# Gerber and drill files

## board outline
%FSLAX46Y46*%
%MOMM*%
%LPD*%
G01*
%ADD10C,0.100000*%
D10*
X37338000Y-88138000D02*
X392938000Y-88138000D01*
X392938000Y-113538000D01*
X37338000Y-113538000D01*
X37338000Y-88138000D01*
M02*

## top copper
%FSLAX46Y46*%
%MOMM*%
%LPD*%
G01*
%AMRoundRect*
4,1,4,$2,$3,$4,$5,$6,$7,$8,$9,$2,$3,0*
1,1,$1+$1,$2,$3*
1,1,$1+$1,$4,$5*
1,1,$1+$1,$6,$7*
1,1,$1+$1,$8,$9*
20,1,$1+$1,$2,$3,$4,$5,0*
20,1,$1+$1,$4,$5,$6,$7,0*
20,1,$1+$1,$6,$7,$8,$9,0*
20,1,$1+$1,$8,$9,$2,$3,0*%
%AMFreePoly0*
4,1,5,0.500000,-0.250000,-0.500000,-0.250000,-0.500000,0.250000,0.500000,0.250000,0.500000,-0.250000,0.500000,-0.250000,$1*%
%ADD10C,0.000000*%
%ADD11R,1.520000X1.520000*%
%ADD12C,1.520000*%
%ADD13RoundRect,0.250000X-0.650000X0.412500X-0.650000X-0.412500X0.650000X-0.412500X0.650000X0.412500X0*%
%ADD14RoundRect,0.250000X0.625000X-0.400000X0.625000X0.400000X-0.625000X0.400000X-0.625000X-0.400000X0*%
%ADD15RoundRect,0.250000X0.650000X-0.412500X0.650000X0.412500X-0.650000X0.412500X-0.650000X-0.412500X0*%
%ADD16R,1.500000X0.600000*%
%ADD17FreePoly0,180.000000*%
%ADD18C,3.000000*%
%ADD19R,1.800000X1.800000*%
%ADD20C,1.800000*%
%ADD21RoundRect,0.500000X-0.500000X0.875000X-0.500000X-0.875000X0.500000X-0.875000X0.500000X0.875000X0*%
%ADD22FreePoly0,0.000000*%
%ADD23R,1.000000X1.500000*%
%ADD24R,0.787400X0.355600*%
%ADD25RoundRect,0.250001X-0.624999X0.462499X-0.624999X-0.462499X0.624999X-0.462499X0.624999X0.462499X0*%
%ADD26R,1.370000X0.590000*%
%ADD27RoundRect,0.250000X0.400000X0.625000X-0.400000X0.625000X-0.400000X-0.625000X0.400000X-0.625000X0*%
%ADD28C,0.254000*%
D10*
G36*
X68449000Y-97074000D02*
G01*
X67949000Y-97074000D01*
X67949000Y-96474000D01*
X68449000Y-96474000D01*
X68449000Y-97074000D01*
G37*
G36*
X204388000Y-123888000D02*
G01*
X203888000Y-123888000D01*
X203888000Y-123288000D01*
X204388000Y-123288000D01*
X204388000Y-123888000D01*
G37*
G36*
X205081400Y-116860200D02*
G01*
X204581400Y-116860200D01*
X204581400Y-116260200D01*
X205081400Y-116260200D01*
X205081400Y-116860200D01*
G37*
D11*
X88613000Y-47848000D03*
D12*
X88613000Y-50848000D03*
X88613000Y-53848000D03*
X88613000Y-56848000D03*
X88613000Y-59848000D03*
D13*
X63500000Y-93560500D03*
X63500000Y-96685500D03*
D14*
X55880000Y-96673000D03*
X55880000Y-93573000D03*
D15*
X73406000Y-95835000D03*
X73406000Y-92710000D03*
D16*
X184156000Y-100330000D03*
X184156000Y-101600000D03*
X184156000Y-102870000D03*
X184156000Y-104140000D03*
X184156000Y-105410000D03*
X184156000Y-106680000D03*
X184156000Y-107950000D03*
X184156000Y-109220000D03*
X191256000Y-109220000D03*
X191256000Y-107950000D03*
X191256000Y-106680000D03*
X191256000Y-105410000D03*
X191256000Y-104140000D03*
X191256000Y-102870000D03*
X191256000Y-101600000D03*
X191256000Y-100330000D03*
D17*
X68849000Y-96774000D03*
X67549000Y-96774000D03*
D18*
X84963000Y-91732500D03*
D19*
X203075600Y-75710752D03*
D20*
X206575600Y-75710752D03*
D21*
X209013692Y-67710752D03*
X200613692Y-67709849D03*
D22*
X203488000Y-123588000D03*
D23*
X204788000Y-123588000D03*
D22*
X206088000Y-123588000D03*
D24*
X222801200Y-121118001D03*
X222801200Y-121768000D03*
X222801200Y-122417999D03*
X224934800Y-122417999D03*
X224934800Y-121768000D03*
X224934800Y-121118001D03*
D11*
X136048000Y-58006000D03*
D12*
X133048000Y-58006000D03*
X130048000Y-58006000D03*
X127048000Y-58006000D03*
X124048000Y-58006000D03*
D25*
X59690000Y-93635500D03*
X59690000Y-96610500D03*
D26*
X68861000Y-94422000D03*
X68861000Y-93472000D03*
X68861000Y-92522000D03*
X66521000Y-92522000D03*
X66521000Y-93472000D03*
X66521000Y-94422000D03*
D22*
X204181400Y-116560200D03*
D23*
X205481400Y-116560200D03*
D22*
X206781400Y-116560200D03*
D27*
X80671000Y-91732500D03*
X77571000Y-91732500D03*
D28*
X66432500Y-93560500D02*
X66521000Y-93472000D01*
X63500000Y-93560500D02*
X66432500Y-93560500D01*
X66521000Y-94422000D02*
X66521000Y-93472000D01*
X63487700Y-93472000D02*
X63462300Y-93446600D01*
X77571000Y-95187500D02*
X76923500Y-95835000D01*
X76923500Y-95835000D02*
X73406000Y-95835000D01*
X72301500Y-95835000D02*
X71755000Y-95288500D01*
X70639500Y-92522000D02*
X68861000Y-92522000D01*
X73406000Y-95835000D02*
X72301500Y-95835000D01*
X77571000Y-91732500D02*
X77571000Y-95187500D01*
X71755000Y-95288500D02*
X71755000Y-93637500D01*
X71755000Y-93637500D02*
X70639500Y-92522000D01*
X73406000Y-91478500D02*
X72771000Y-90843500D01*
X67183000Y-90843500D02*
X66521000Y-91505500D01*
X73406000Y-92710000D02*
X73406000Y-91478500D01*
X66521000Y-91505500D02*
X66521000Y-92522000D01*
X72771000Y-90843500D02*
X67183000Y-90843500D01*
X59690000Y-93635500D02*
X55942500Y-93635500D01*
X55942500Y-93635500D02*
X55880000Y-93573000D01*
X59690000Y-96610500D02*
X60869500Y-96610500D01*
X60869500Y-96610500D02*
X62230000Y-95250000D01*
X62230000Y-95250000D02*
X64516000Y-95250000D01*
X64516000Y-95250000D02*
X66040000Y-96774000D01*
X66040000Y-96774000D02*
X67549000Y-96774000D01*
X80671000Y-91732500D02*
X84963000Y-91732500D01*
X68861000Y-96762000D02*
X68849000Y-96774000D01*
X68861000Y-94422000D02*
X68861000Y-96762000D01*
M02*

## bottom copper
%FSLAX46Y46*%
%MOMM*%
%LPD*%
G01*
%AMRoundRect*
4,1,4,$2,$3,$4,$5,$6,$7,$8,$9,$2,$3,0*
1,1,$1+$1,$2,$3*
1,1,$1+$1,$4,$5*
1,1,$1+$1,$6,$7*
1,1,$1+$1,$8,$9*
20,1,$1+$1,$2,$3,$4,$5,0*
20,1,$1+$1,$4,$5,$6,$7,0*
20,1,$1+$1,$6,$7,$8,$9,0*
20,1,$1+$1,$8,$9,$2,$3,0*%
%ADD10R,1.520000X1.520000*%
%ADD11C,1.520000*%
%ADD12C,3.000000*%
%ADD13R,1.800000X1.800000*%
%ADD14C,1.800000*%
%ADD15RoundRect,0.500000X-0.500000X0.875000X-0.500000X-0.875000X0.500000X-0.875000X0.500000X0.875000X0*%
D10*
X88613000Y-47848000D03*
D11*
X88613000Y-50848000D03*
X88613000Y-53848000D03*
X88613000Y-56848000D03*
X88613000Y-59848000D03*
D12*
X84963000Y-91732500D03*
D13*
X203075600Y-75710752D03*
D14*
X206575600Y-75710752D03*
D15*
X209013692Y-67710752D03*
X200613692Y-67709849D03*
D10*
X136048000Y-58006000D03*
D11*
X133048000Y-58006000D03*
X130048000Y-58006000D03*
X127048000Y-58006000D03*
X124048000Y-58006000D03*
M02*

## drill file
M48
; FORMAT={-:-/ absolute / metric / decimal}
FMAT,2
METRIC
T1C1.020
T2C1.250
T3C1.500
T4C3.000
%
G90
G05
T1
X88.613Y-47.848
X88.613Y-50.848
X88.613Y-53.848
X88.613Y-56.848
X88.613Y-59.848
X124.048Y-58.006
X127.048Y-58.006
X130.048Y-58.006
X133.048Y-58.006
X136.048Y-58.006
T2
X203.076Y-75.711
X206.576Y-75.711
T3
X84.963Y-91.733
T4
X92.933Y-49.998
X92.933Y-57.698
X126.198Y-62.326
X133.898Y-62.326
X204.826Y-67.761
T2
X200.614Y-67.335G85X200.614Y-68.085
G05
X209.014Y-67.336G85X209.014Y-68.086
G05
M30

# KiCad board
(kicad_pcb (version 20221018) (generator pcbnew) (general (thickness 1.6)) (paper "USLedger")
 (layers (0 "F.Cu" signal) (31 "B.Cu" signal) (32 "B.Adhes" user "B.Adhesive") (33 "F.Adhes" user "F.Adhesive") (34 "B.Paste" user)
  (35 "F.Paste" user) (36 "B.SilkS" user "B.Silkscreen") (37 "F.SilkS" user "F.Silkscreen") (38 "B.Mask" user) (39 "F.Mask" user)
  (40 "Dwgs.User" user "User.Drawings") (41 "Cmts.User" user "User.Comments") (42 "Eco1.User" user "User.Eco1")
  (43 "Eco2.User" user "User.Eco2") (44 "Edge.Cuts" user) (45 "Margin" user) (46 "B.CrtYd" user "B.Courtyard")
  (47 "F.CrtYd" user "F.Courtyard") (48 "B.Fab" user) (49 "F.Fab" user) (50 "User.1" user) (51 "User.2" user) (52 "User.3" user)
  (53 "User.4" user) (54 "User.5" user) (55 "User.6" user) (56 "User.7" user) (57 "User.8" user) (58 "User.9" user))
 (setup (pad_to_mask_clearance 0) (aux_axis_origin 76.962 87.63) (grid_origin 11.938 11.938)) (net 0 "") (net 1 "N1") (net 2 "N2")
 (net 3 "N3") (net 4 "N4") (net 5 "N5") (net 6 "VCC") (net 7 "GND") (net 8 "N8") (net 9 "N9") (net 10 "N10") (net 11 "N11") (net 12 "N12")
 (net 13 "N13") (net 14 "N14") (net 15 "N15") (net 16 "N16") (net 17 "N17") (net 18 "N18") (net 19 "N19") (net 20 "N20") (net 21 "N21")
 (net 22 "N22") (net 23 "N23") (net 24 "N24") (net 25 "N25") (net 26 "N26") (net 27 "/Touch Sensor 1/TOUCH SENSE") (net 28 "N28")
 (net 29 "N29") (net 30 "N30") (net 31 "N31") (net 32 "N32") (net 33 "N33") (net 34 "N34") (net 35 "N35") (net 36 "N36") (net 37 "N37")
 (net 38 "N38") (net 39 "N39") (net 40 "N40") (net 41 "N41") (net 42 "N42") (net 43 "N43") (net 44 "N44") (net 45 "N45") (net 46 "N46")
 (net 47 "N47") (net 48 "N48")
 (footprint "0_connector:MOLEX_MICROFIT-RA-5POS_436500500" (layer "F.Cu") (at 88.613 47.848 90)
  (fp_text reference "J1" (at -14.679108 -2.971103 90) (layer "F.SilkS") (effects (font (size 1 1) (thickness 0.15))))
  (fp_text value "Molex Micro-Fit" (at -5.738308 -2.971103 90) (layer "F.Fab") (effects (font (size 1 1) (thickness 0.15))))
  (pad "" np_thru_hole circle (at -9.85 4.32 90) (size 3 3) (drill 3) (layers "*.Cu" "*.Mask"))
  (pad "" np_thru_hole circle (at -2.15 4.32 90) (size 3 3) (drill 3) (layers "*.Cu" "*.Mask"))
  (pad "1" thru_hole rect (at 0 0 90) (size 1.52 1.52) (drill 1.02) (layers "*.Cu") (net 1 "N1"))
  (pad "2" thru_hole circle (at -3 0 90) (size 1.52 1.52) (drill 1.02) (layers "*.Cu") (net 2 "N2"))
  (pad "3" thru_hole circle (at -6 0 90) (size 1.52 1.52) (drill 1.02) (layers "*.Cu") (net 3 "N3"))
  (pad "4" thru_hole circle (at -9 0 90) (size 1.52 1.52) (drill 1.02) (layers "*.Cu") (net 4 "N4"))
  (pad "5" thru_hole circle (at -12 0 90) (size 1.52 1.52) (drill 1.02) (layers "*.Cu") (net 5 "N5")))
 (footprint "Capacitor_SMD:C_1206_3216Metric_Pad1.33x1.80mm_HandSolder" (layer "F.Cu") (at 63.5 95.123 -90)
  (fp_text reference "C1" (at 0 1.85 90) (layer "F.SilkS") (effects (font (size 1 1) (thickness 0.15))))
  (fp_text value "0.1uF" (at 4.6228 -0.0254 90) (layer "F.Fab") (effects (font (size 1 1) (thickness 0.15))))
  (pad "1" smd roundrect (at -1.5625 0 270) (size 1.325 1.8) (layers "F.Cu" "F.Paste" "F.Mask") (roundrect_rratio 0.188679) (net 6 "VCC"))
  (pad "2" smd roundrect (at 1.5625 0 270) (size 1.325 1.8) (layers "F.Cu" "F.Paste" "F.Mask") (roundrect_rratio 0.188679) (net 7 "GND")))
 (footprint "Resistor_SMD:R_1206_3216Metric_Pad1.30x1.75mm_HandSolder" (layer "F.Cu") (at 55.88 95.123 90)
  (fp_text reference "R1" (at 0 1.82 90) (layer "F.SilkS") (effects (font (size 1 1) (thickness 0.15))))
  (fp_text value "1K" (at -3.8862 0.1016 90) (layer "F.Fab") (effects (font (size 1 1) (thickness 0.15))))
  (pad "1" smd roundrect (at -1.55 0 90) (size 1.3 1.75) (layers "F.Cu" "F.Paste" "F.Mask") (roundrect_rratio 0.192308) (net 7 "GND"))
  (pad "2" smd roundrect (at 1.55 0 90) (size 1.3 1.75) (layers "F.Cu" "F.Paste" "F.Mask") (roundrect_rratio 0.192308) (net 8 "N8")))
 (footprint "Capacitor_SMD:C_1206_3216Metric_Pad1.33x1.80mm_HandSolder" (layer "F.Cu") (at 73.406 94.2725 90)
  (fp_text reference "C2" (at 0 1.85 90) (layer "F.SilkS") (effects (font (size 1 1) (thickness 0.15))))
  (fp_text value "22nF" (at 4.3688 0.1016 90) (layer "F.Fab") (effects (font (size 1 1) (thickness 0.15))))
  (pad "1" smd roundrect (at -1.5625 0 90) (size 1.325 1.8) (layers "F.Cu" "F.Paste" "F.Mask") (roundrect_rratio 0.188679) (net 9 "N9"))
  (pad "2" smd roundrect (at 1.5625 0 90) (size 1.325 1.8) (layers "F.Cu" "F.Paste" "F.Mask") (roundrect_rratio 0.188679) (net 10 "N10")))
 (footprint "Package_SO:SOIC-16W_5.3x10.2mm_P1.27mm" (layer "F.Cu") (at 187.706 104.775)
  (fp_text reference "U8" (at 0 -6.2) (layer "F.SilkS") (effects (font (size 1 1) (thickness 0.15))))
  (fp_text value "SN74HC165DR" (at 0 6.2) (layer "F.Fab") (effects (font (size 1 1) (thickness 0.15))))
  (pad "1" smd rect (at -3.55 -4.445) (size 1.5 0.6) (layers "F.Cu" "F.Paste" "F.Mask") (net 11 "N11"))
  (pad "2" smd rect (at -3.55 -3.175) (size 1.5 0.6) (layers "F.Cu" "F.Paste" "F.Mask") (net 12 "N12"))
  (pad "3" smd rect (at -3.55 -1.905) (size 1.5 0.6) (layers "F.Cu" "F.Paste" "F.Mask") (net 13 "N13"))
  (pad "4" smd rect (at -3.55 -0.635) (size 1.5 0.6) (layers "F.Cu" "F.Paste" "F.Mask") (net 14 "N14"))
  (pad "5" smd rect (at -3.55 0.635) (size 1.5 0.6) (layers "F.Cu" "F.Paste" "F.Mask") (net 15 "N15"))
  (pad "6" smd rect (at -3.55 1.905) (size 1.5 0.6) (layers "F.Cu" "F.Paste" "F.Mask") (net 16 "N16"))
  (pad "7" smd rect (at -3.55 3.175) (size 1.5 0.6) (layers "F.Cu" "F.Paste" "F.Mask") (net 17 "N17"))
  (pad "8" smd rect (at -3.55 4.445) (size 1.5 0.6) (layers "F.Cu" "F.Paste" "F.Mask") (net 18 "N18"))
  (pad "9" smd rect (at 3.55 4.445) (size 1.5 0.6) (layers "F.Cu" "F.Paste" "F.Mask") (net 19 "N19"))
  (pad "10" smd rect (at 3.55 3.175) (size 1.5 0.6) (layers "F.Cu" "F.Paste" "F.Mask") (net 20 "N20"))
  (pad "11" smd rect (at 3.55 1.905) (size 1.5 0.6) (layers "F.Cu" "F.Paste" "F.Mask") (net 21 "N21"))
  (pad "12" smd rect (at 3.55 0.635) (size 1.5 0.6) (layers "F.Cu" "F.Paste" "F.Mask") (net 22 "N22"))
  (pad "13" smd rect (at 3.55 -0.635) (size 1.5 0.6) (layers "F.Cu" "F.Paste" "F.Mask") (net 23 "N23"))
  (pad "14" smd rect (at 3.55 -1.905) (size 1.5 0.6) (layers "F.Cu" "F.Paste" "F.Mask") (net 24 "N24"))
  (pad "15" smd rect (at 3.55 -3.175) (size 1.5 0.6) (layers "F.Cu" "F.Paste" "F.Mask") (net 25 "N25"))
  (pad "16" smd rect (at 3.55 -4.445) (size 1.5 0.6) (layers "F.Cu" "F.Paste" "F.Mask") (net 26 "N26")))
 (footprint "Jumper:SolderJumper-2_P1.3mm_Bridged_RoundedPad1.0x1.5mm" (layer "F.Cu") (at 68.199 96.774 180) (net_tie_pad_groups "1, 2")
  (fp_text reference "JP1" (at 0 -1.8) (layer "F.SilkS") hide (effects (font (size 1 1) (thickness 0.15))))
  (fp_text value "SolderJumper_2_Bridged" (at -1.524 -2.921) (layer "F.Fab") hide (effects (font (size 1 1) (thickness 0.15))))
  (fp_poly (pts (xy 0.25 -0.3) (xy -0.25 -0.3) (xy -0.25 0.3) (xy 0.25 0.3)) (stroke (width 0) (type solid)) (fill solid) (layer "F.Cu"))
  (pad "1" smd custom (at -0.65 0 180) (size 1 0.5) (layers "F.Cu" "F.Mask") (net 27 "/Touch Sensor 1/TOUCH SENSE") (zone_connect 2)
   (options (clearance outline) (anchor rect)) (primitives))
  (pad "2" smd custom (at 0.65 0 180) (size 1 0.5) (layers "F.Cu" "F.Mask") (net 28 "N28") (zone_connect 2)
   (options (clearance outline) (anchor rect)) (primitives)))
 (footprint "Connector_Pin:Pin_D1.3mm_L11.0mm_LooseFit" (layer "F.Cu") (at 84.963 91.7325)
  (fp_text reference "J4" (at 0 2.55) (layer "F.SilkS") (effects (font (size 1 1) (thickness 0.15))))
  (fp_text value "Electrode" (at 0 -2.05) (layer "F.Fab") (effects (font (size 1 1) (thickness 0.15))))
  (pad "1" thru_hole circle (at 0 0) (size 3 3) (drill 1.5) (layers "*.Cu" "*.Mask") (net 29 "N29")))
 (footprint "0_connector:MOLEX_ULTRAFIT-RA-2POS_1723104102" (layer "F.Cu") (at 204.613692 80.359849)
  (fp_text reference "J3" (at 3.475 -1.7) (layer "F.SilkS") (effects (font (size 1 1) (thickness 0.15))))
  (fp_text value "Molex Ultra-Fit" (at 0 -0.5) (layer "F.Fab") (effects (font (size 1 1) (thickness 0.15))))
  (pad "" np_thru_hole circle (at 0.211908 -12.599097 180) (size 3 3) (drill 3) (layers "*.Cu" "*.Mask"))
  (pad "1" thru_hole rect (at -1.538092 -4.649097 180) (size 1.8 1.8) (drill 1.25) (layers "*.Cu" "*.Mask") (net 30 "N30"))
  (pad "2" thru_hole circle (at 1.961908 -4.649097 180) (size 1.8 1.8) (drill 1.25) (layers "*.Cu" "*.Mask") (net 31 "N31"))
  (pad "3" thru_hole roundrect (at 4.4 -12.649097 270) (size 2.75 2) (drill oval 2 1.25) (layers "*.Cu" "*.Mask") (roundrect_rratio 0.25))
  (pad "4" thru_hole roundrect (at -4 -12.65 270) (size 2.75 2) (drill oval 2 1.25) (layers "*.Cu" "*.Mask") (roundrect_rratio 0.25)))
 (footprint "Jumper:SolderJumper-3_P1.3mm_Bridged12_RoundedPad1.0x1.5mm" (layer "F.Cu") (at 204.788 123.588) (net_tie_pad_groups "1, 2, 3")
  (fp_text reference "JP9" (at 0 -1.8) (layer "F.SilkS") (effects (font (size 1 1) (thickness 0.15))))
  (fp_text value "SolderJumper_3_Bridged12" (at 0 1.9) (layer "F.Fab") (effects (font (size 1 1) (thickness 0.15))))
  (fp_poly (pts (xy -0.9 -0.3) (xy -0.4 -0.3) (xy -0.4 0.3) (xy -0.9 0.3)) (stroke (width 0) (type solid)) (fill solid) (layer "F.Cu"))
  (pad "1" smd custom (at -1.3 0) (size 1 0.5) (layers "F.Cu" "F.Mask") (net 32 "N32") (zone_connect 2)
   (options (clearance outline) (anchor rect)) (primitives))
  (pad "2" smd rect (at 0 0) (size 1 1.5) (layers "F.Cu" "F.Mask") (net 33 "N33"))
  (pad "3" smd custom (at 1.3 0) (size 1 0.5) (layers "F.Cu" "F.Mask") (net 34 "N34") (zone_connect 2)
   (options (clearance outline) (anchor rect)) (primitives)))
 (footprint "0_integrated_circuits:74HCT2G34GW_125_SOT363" (layer "F.Cu") (at 223.868 121.768)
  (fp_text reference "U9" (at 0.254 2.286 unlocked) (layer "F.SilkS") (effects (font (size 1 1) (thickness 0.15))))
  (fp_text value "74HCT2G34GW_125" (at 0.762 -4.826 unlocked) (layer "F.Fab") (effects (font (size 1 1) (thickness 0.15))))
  (pad "1" smd rect (at -1.0668 -0.649999) (size 0.7874 0.3556) (layers "F.Cu" "F.Paste" "F.Mask") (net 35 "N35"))
  (pad "2" smd rect (at -1.0668 0) (size 0.7874 0.3556) (layers "F.Cu" "F.Paste" "F.Mask") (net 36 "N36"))
  (pad "3" smd rect (at -1.0668 0.649999) (size 0.7874 0.3556) (layers "F.Cu" "F.Paste" "F.Mask") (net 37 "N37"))
  (pad "4" smd rect (at 1.0668 0.649999) (size 0.7874 0.3556) (layers "F.Cu" "F.Paste" "F.Mask") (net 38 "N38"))
  (pad "5" smd rect (at 1.0668 0) (size 0.7874 0.3556) (layers "F.Cu" "F.Paste" "F.Mask") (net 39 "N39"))
  (pad "6" smd rect (at 1.0668 -0.649999) (size 0.7874 0.3556) (layers "F.Cu" "F.Paste" "F.Mask") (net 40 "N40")))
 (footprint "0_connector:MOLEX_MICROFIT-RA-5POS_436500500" (layer "F.Cu") (at 136.048 58.006)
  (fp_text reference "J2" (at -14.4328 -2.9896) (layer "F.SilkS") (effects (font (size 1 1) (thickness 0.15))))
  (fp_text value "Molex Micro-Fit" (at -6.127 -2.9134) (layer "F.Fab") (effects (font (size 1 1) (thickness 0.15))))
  (pad "" np_thru_hole circle (at -9.85 4.32) (size 3 3) (drill 3) (layers "*.Cu" "*.Mask"))
  (pad "" np_thru_hole circle (at -2.15 4.32) (size 3 3) (drill 3) (layers "*.Cu" "*.Mask"))
  (pad "1" thru_hole rect (at 0 0) (size 1.52 1.52) (drill 1.02) (layers "*.Cu") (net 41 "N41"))
  (pad "2" thru_hole circle (at -3 0) (size 1.52 1.52) (drill 1.02) (layers "*.Cu") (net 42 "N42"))
  (pad "3" thru_hole circle (at -6 0) (size 1.52 1.52) (drill 1.02) (layers "*.Cu") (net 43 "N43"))
  (pad "4" thru_hole circle (at -9 0) (size 1.52 1.52) (drill 1.02) (layers "*.Cu") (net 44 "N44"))
  (pad "5" thru_hole circle (at -12 0) (size 1.52 1.52) (drill 1.02) (layers "*.Cu") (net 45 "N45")))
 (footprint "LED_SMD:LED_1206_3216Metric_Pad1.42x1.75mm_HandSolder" (layer "F.Cu") (at 59.69 95.123 -90)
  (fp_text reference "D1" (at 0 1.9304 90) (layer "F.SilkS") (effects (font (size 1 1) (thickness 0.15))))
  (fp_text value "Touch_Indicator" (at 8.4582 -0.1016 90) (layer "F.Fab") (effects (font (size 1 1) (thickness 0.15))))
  (pad "1" smd roundrect (at -1.4875 0 270) (size 1.425 1.75) (layers "F.Cu" "F.Paste" "F.Mask") (roundrect_rratio 0.175439) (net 8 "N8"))
  (pad "2" smd roundrect (at 1.4875 0 270) (size 1.425 1.75) (layers "F.Cu" "F.Paste" "F.Mask") (roundrect_rratio 0.175439) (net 28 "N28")))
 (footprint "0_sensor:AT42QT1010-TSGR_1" (layer "F.Cu") (at 67.691 93.472 180)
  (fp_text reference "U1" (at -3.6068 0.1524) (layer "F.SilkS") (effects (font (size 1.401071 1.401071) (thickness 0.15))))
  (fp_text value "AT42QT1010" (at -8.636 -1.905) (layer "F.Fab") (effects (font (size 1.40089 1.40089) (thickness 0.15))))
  (pad "1" smd rect (at -1.17 -0.95 180) (size 1.37 0.59) (layers "F.Cu" "F.Paste" "F.Mask") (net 27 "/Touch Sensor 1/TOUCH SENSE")
   (solder_mask_margin 0.102))
  (pad "2" smd rect (at -1.17 0 180) (size 1.37 0.59) (layers "F.Cu" "F.Paste" "F.Mask") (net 7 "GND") (solder_mask_margin 0.102))
  (pad "3" smd rect (at -1.17 0.95 180) (size 1.37 0.59) (layers "F.Cu" "F.Paste" "F.Mask") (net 9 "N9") (solder_mask_margin 0.102))
  (pad "4" smd rect (at 1.17 0.95 180) (size 1.37 0.59) (layers "F.Cu" "F.Paste" "F.Mask") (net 10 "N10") (solder_mask_margin 0.102))
  (pad "5" smd rect (at 1.17 0 180) (size 1.37 0.59) (layers "F.Cu" "F.Paste" "F.Mask") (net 6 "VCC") (solder_mask_margin 0.102))
  (pad "6" smd rect (at 1.17 -0.95 180) (size 1.37 0.59) (layers "F.Cu" "F.Paste" "F.Mask") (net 6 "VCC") (solder_mask_margin 0.102)))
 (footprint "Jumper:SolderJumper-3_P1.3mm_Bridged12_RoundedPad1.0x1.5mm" (layer "F.Cu") (at 205.4814 116.5602)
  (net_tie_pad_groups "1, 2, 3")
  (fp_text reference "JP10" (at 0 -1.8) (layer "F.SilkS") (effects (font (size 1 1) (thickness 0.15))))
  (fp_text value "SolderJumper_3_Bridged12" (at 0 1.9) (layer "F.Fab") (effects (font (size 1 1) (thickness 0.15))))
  (fp_poly (pts (xy -0.9 -0.3) (xy -0.4 -0.3) (xy -0.4 0.3) (xy -0.9 0.3)) (stroke (width 0) (type solid)) (fill solid) (layer "F.Cu"))
  (pad "1" smd custom (at -1.3 0) (size 1 0.5) (layers "F.Cu" "F.Mask") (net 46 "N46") (zone_connect 2)
   (options (clearance outline) (anchor rect)) (primitives))
  (pad "2" smd rect (at 0 0) (size 1 1.5) (layers "F.Cu" "F.Mask") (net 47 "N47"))
  (pad "3" smd custom (at 1.3 0) (size 1 0.5) (layers "F.Cu" "F.Mask") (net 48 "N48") (zone_connect 2)
   (options (clearance outline) (anchor rect)) (primitives)))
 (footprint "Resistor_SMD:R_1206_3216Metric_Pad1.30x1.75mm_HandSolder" (layer "F.Cu") (at 79.121 91.7325 180)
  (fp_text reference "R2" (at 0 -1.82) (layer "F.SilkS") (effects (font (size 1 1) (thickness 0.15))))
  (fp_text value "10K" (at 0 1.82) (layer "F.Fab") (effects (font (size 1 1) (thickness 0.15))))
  (pad "1" smd roundrect (at -1.55 0 180) (size 1.3 1.75) (layers "F.Cu" "F.Paste" "F.Mask") (roundrect_rratio 0.192308) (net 29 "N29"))
  (pad "2" smd roundrect (at 1.55 0 180) (size 1.3 1.75) (layers "F.Cu" "F.Paste" "F.Mask") (roundrect_rratio 0.192308) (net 9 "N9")))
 (gr_rect (start 37.338 88.138) (end 392.938 113.538) (stroke (width 0.1) (type default)) (fill none) (layer "Edge.Cuts"))
 (segment (start 66.4325 93.5605) (end 66.521 93.472) (width 0.254) (layer "F.Cu") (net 6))
 (segment (start 63.5 93.5605) (end 66.4325 93.5605) (width 0.254) (layer "F.Cu") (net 6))
 (segment (start 66.521 94.422) (end 66.521 93.472) (width 0.254) (layer "F.Cu") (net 6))
 (segment (start 63.4877 93.472) (end 63.4623 93.4466) (width 0.254) (layer "F.Cu") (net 6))
 (segment (start 77.571 95.1875) (end 76.9235 95.835) (width 0.254) (layer "F.Cu") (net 9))
 (segment (start 76.9235 95.835) (end 73.406 95.835) (width 0.254) (layer "F.Cu") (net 9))
 (segment (start 72.3015 95.835) (end 71.755 95.2885) (width 0.254) (layer "F.Cu") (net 9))
 (segment (start 70.6395 92.522) (end 68.861 92.522) (width 0.254) (layer "F.Cu") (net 9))
 (segment (start 73.406 95.835) (end 72.3015 95.835) (width 0.254) (layer "F.Cu") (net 9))
 (segment (start 77.571 91.7325) (end 77.571 95.1875) (width 0.254) (layer "F.Cu") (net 9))
 (segment (start 71.755 95.2885) (end 71.755 93.6375) (width 0.254) (layer "F.Cu") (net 9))
 (segment (start 71.755 93.6375) (end 70.6395 92.522) (width 0.254) (layer "F.Cu") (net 9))
 (segment (start 73.406 91.4785) (end 72.771 90.8435) (width 0.254) (layer "F.Cu") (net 10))
 (segment (start 67.183 90.8435) (end 66.521 91.5055) (width 0.254) (layer "F.Cu") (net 10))
 (segment (start 73.406 92.71) (end 73.406 91.4785) (width 0.254) (layer "F.Cu") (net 10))
 (segment (start 66.521 91.5055) (end 66.521 92.522) (width 0.254) (layer "F.Cu") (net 10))
 (segment (start 72.771 90.8435) (end 67.183 90.8435) (width 0.254) (layer "F.Cu") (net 10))
 (segment (start 59.69 93.6355) (end 55.9425 93.6355) (width 0.254) (layer "F.Cu") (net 8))
 (segment (start 55.9425 93.6355) (end 55.88 93.573) (width 0.254) (layer "F.Cu") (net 8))
 (segment (start 59.69 96.6105) (end 60.8695 96.6105) (width 0.254) (layer "F.Cu") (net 28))
 (segment (start 60.8695 96.6105) (end 62.23 95.25) (width 0.254) (layer "F.Cu") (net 28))
 (segment (start 62.23 95.25) (end 64.516 95.25) (width 0.254) (layer "F.Cu") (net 28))
 (segment (start 64.516 95.25) (end 66.04 96.774) (width 0.254) (layer "F.Cu") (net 28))
 (segment (start 66.04 96.774) (end 67.549 96.774) (width 0.254) (layer "F.Cu") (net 28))
 (segment (start 80.671 91.7325) (end 84.963 91.7325) (width 0.254) (layer "F.Cu") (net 29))
 (segment (start 68.861 96.762) (end 68.849 96.774) (width 0.254) (layer "F.Cu") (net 27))
 (segment (start 68.861 94.422) (end 68.861 96.762) (width 0.254) (layer "F.Cu") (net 27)))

